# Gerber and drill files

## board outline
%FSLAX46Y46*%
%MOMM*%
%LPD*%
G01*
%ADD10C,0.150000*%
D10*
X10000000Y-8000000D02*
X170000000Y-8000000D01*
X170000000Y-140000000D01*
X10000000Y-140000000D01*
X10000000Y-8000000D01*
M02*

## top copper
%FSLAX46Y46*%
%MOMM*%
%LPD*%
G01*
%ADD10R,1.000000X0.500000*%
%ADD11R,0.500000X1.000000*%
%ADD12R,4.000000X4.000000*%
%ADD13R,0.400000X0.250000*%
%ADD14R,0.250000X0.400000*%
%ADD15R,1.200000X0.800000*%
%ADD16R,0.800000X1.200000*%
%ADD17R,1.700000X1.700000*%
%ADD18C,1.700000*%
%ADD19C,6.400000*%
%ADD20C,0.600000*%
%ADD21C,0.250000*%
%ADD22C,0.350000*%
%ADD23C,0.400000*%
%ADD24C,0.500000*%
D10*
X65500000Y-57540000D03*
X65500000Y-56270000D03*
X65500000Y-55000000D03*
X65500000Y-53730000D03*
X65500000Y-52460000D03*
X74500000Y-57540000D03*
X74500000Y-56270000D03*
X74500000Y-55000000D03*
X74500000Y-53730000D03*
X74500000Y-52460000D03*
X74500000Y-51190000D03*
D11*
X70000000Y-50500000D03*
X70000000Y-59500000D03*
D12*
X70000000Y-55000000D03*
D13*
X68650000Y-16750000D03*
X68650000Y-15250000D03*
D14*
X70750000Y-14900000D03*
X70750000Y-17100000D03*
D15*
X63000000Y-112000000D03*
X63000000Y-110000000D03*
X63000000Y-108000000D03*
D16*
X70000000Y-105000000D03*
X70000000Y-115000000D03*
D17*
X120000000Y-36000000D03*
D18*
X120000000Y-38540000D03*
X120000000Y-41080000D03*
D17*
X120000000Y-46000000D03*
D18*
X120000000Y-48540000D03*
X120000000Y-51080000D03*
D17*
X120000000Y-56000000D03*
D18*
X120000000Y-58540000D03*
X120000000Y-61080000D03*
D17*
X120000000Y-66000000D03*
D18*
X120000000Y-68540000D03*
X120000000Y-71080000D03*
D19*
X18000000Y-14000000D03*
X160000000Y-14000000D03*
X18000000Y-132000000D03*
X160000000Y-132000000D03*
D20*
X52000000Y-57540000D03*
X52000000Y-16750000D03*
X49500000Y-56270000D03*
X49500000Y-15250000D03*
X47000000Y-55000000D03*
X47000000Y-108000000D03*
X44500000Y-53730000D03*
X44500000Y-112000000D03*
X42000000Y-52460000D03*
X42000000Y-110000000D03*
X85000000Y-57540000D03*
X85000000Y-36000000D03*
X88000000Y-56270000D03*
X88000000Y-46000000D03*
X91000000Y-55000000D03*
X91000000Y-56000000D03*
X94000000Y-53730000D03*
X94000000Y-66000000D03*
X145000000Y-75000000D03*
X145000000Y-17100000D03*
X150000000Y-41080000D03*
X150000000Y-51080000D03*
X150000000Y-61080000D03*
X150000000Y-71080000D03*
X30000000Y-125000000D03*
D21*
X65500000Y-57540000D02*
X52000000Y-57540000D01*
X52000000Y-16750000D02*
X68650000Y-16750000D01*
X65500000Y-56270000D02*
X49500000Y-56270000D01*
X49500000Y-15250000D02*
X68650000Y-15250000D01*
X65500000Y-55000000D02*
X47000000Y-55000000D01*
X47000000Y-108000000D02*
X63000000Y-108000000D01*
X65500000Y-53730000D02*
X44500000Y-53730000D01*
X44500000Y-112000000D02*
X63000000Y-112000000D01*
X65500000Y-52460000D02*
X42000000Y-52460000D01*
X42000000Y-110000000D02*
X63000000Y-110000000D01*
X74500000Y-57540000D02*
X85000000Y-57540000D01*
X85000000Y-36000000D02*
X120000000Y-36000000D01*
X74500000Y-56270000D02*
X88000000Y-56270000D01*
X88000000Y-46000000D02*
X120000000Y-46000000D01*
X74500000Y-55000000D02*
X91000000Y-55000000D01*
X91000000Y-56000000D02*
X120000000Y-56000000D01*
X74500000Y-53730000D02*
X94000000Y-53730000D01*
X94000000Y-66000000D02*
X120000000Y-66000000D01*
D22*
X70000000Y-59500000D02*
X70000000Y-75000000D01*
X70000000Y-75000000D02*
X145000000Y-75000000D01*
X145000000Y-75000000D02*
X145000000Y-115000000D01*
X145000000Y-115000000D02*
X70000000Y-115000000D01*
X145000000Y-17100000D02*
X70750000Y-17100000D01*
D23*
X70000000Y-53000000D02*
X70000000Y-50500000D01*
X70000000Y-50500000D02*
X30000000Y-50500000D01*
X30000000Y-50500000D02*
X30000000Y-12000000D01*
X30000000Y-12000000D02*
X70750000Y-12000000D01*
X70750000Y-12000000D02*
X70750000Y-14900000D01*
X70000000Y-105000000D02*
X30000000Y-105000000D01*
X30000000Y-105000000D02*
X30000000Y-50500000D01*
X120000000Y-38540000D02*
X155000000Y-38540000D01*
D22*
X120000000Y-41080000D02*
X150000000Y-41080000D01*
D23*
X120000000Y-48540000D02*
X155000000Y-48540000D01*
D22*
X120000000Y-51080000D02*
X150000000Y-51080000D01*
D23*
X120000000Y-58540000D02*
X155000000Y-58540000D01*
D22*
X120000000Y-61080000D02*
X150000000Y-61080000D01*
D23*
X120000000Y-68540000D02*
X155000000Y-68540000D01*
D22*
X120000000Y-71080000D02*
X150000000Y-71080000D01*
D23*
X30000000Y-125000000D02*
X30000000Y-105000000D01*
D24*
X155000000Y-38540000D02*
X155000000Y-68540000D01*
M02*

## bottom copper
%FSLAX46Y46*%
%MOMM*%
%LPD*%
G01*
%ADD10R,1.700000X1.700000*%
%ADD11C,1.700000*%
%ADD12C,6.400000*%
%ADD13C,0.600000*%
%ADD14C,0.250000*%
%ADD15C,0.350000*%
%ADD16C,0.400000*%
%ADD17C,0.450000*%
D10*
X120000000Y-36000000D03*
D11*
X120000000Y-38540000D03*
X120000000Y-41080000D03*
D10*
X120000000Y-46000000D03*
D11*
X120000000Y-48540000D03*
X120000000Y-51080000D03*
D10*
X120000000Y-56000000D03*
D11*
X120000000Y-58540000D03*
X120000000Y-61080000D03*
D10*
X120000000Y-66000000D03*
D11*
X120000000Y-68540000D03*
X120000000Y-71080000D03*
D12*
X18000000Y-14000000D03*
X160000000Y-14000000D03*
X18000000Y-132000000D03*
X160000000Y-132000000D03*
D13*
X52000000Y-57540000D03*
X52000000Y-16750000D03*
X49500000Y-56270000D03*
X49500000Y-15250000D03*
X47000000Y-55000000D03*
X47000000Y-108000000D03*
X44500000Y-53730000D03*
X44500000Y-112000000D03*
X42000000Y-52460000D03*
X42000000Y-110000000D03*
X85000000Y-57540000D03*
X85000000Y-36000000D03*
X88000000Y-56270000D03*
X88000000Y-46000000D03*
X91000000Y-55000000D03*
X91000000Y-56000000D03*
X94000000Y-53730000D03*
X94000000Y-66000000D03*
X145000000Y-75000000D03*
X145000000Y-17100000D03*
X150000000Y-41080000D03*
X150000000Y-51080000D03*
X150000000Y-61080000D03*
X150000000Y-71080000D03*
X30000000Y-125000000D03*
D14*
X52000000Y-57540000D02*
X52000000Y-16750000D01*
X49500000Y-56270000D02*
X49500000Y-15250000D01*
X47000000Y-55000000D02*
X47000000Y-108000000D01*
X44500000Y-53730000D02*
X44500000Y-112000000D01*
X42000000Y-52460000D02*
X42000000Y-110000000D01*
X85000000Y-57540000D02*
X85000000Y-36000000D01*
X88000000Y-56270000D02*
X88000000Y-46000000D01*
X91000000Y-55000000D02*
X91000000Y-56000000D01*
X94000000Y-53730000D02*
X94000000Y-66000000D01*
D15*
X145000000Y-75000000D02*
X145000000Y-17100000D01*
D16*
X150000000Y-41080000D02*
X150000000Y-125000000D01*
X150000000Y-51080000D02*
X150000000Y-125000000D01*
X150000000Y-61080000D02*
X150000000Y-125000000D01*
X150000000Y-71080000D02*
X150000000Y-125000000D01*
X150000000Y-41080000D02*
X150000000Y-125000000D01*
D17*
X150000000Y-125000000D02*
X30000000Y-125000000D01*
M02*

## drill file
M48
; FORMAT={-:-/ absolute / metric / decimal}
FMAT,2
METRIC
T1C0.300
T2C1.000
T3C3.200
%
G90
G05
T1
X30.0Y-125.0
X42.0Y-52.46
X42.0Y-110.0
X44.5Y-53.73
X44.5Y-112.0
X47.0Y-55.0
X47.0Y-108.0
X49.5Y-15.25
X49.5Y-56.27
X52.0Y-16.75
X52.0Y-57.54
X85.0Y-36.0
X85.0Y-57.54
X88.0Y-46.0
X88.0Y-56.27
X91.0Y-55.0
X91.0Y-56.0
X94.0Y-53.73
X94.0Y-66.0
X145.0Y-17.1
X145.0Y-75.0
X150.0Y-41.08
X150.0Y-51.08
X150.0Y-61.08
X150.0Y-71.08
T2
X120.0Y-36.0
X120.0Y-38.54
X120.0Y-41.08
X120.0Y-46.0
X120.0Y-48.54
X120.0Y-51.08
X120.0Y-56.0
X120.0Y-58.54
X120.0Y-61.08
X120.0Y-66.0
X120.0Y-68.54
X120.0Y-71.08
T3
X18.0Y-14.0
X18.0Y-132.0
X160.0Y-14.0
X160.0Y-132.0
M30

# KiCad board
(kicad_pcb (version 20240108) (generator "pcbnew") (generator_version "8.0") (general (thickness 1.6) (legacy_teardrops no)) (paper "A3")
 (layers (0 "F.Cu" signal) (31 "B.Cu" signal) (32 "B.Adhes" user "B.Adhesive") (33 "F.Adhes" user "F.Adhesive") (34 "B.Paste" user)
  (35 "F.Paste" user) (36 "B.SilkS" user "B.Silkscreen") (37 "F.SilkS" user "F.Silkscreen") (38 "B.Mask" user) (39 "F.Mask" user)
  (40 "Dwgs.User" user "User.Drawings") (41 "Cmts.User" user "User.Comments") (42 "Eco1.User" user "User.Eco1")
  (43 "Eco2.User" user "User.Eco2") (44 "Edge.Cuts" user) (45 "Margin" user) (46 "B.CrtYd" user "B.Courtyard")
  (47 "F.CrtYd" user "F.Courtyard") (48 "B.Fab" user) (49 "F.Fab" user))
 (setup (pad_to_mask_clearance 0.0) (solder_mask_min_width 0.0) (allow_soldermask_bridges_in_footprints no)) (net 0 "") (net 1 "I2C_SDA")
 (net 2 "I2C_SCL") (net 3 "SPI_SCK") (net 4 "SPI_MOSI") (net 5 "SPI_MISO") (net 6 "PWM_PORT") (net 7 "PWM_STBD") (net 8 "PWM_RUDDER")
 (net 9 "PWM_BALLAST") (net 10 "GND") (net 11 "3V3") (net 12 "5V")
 (gr_rect (start 10 8) (end 170 140) (stroke (width 0.15) (type solid)) (fill none) (layer "Edge.Cuts"))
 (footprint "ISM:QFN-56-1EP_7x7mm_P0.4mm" (layer "F.Cu") (at 70 55)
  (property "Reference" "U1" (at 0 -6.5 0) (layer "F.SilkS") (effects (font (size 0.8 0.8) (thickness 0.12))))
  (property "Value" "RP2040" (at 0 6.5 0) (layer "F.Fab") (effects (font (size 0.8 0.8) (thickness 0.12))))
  (pad "1" smd rect (at -4.5 2.54) (size 1.0 0.5) (layers "F.Cu" "F.Paste" "F.Mask") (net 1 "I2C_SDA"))
  (pad "2" smd rect (at -4.5 1.27) (size 1.0 0.5) (layers "F.Cu" "F.Paste" "F.Mask") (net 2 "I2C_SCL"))
  (pad "3" smd rect (at -4.5 0) (size 1.0 0.5) (layers "F.Cu" "F.Paste" "F.Mask") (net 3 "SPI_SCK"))
  (pad "4" smd rect (at -4.5 -1.27) (size 1.0 0.5) (layers "F.Cu" "F.Paste" "F.Mask") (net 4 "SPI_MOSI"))
  (pad "5" smd rect (at -4.5 -2.54) (size 1.0 0.5) (layers "F.Cu" "F.Paste" "F.Mask") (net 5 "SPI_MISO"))
  (pad "6" smd rect (at 4.5 2.54) (size 1.0 0.5) (layers "F.Cu" "F.Paste" "F.Mask") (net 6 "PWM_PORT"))
  (pad "7" smd rect (at 4.5 1.27) (size 1.0 0.5) (layers "F.Cu" "F.Paste" "F.Mask") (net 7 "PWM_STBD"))
  (pad "8" smd rect (at 4.5 0) (size 1.0 0.5) (layers "F.Cu" "F.Paste" "F.Mask") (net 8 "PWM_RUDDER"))
  (pad "9" smd rect (at 4.5 -1.27) (size 1.0 0.5) (layers "F.Cu" "F.Paste" "F.Mask") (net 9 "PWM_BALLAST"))
  (pad "12" smd rect (at 4.5 -2.54) (size 1.0 0.5) (layers "F.Cu" "F.Paste" "F.Mask"))
  (pad "13" smd rect (at 4.5 -3.81) (size 1.0 0.5) (layers "F.Cu" "F.Paste" "F.Mask"))
  (pad "10" smd rect (at 0 -4.5) (size 0.5 1.0) (layers "F.Cu" "F.Paste" "F.Mask") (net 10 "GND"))
  (pad "11" smd rect (at 0 4.5) (size 0.5 1.0) (layers "F.Cu" "F.Paste" "F.Mask") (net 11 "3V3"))
  (pad "EP" smd rect (at 0 0) (size 4 4) (layers "F.Cu" "F.Paste" "F.Mask") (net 10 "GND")))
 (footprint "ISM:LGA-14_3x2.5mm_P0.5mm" (layer "F.Cu") (at 70 16)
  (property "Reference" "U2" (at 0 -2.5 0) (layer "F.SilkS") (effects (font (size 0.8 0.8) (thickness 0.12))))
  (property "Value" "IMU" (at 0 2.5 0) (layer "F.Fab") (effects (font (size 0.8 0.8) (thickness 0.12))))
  (pad "1" smd rect (at -1.35 0.75) (size 0.4 0.25) (layers "F.Cu" "F.Paste" "F.Mask") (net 1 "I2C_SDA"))
  (pad "2" smd rect (at -1.35 -0.75) (size 0.4 0.25) (layers "F.Cu" "F.Paste" "F.Mask") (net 2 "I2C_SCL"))
  (pad "3" smd rect (at 0.75 -1.1) (size 0.25 0.4) (layers "F.Cu" "F.Paste" "F.Mask") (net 10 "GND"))
  (pad "4" smd rect (at 0.75 1.1) (size 0.25 0.4) (layers "F.Cu" "F.Paste" "F.Mask") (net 11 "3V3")))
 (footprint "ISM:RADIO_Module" (layer "F.Cu") (at 70 110)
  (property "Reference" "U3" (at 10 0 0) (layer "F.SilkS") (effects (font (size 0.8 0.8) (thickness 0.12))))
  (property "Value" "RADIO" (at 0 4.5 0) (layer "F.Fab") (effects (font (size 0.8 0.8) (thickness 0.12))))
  (pad "1" smd rect (at -7 2) (size 1.2 0.8) (layers "F.Cu" "F.Paste" "F.Mask") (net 4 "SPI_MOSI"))
  (pad "2" smd rect (at -7 0) (size 1.2 0.8) (layers "F.Cu" "F.Paste" "F.Mask") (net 5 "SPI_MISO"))
  (pad "3" smd rect (at -7 -2) (size 1.2 0.8) (layers "F.Cu" "F.Paste" "F.Mask") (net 3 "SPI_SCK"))
  (pad "4" smd rect (at 0 -5) (size 0.8 1.2) (layers "F.Cu" "F.Paste" "F.Mask") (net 10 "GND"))
  (pad "5" smd rect (at 0 5) (size 0.8 1.2) (layers "F.Cu" "F.Paste" "F.Mask") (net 11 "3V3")))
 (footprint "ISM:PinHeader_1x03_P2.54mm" (layer "F.Cu") (at 120 36)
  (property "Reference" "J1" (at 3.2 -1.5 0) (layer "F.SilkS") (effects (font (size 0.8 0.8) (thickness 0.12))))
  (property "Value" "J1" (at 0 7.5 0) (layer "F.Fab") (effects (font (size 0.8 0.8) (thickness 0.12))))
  (pad "1" thru_hole rect (at 0 0) (size 1.7 1.7) (drill 1.0) (layers "*.Cu" "*.Mask") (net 6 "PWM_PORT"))
  (pad "2" thru_hole circle (at 0 2.54) (size 1.7 1.7) (drill 1.0) (layers "*.Cu" "*.Mask") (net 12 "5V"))
  (pad "3" thru_hole circle (at 0 5.08) (size 1.7 1.7) (drill 1.0) (layers "*.Cu" "*.Mask") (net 10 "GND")))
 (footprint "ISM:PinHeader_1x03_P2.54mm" (layer "F.Cu") (at 120 46)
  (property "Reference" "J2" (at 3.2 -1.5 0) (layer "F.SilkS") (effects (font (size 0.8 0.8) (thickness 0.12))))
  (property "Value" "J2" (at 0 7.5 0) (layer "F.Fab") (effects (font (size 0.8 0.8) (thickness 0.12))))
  (pad "1" thru_hole rect (at 0 0) (size 1.7 1.7) (drill 1.0) (layers "*.Cu" "*.Mask") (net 7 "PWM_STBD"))
  (pad "2" thru_hole circle (at 0 2.54) (size 1.7 1.7) (drill 1.0) (layers "*.Cu" "*.Mask") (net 12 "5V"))
  (pad "3" thru_hole circle (at 0 5.08) (size 1.7 1.7) (drill 1.0) (layers "*.Cu" "*.Mask") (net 10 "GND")))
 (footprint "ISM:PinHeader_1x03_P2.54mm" (layer "F.Cu") (at 120 56)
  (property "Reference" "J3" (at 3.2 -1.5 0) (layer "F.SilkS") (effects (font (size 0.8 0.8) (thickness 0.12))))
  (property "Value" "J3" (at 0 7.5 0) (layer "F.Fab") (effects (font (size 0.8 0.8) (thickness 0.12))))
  (pad "1" thru_hole rect (at 0 0) (size 1.7 1.7) (drill 1.0) (layers "*.Cu" "*.Mask") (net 8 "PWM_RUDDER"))
  (pad "2" thru_hole circle (at 0 2.54) (size 1.7 1.7) (drill 1.0) (layers "*.Cu" "*.Mask") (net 12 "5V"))
  (pad "3" thru_hole circle (at 0 5.08) (size 1.7 1.7) (drill 1.0) (layers "*.Cu" "*.Mask") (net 10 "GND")))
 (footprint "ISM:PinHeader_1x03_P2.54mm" (layer "F.Cu") (at 120 66)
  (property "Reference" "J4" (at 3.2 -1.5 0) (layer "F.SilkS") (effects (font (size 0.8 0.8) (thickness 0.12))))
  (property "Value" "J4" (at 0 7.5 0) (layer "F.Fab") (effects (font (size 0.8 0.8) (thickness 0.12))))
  (pad "1" thru_hole rect (at 0 0) (size 1.7 1.7) (drill 1.0) (layers "*.Cu" "*.Mask") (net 9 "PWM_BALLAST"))
  (pad "2" thru_hole circle (at 0 2.54) (size 1.7 1.7) (drill 1.0) (layers "*.Cu" "*.Mask") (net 12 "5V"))
  (pad "3" thru_hole circle (at 0 5.08) (size 1.7 1.7) (drill 1.0) (layers "*.Cu" "*.Mask") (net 10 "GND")))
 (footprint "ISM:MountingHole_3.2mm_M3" (layer "F.Cu") (at 18 14)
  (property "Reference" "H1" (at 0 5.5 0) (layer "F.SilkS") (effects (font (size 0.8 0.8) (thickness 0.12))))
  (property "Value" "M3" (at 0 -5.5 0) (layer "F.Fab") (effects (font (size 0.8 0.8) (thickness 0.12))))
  (pad "" thru_hole circle (at 0 0) (size 6.4 6.4) (drill 3.2) (layers "*.Cu" "*.Mask")))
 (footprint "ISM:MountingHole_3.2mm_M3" (layer "F.Cu") (at 160 14)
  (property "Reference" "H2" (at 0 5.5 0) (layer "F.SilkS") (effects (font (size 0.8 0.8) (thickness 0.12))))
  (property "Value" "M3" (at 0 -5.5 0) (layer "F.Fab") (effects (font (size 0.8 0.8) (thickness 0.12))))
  (pad "" thru_hole circle (at 0 0) (size 6.4 6.4) (drill 3.2) (layers "*.Cu" "*.Mask")))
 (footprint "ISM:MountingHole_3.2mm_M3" (layer "F.Cu") (at 18 132)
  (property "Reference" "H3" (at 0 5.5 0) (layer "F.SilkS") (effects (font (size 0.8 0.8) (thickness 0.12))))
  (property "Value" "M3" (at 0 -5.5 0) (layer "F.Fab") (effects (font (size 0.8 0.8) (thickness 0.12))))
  (pad "" thru_hole circle (at 0 0) (size 6.4 6.4) (drill 3.2) (layers "*.Cu" "*.Mask")))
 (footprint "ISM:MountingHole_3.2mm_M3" (layer "F.Cu") (at 160 132)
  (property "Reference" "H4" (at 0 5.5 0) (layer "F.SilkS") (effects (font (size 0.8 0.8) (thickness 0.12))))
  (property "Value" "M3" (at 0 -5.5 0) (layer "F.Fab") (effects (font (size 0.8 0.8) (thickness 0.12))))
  (pad "" thru_hole circle (at 0 0) (size 6.4 6.4) (drill 3.2) (layers "*.Cu" "*.Mask")))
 (segment (start 65.5 57.54) (end 52.0 57.54) (width 0.25) (layer "F.Cu") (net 1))
 (segment (start 52.0 57.54) (end 52.0 16.75) (width 0.25) (layer "B.Cu") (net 1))
 (segment (start 52.0 16.75) (end 68.65 16.75) (width 0.25) (layer "F.Cu") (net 1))
 (segment (start 65.5 56.27) (end 49.5 56.27) (width 0.25) (layer "F.Cu") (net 2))
 (segment (start 49.5 56.27) (end 49.5 15.25) (width 0.25) (layer "B.Cu") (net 2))
 (segment (start 49.5 15.25) (end 68.65 15.25) (width 0.25) (layer "F.Cu") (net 2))
 (segment (start 65.5 55) (end 47.0 55) (width 0.25) (layer "F.Cu") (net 3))
 (segment (start 47.0 55) (end 47.0 108) (width 0.25) (layer "B.Cu") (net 3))
 (segment (start 47.0 108) (end 63 108) (width 0.25) (layer "F.Cu") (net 3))
 (segment (start 65.5 53.73) (end 44.5 53.73) (width 0.25) (layer "F.Cu") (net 4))
 (segment (start 44.5 53.73) (end 44.5 112) (width 0.25) (layer "B.Cu") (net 4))
 (segment (start 44.5 112) (end 63 112) (width 0.25) (layer "F.Cu") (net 4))
 (segment (start 65.5 52.46) (end 42.0 52.46) (width 0.25) (layer "F.Cu") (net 5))
 (segment (start 42.0 52.46) (end 42.0 110) (width 0.25) (layer "B.Cu") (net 5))
 (segment (start 42.0 110) (end 63 110) (width 0.25) (layer "F.Cu") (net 5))
 (segment (start 74.5 57.54) (end 85 57.54) (width 0.25) (layer "F.Cu") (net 6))
 (segment (start 85 57.54) (end 85 36) (width 0.25) (layer "B.Cu") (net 6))
 (segment (start 85 36) (end 120 36) (width 0.25) (layer "F.Cu") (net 6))
 (segment (start 74.5 56.27) (end 88 56.27) (width 0.25) (layer "F.Cu") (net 7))
 (segment (start 88 56.27) (end 88 46) (width 0.25) (layer "B.Cu") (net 7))
 (segment (start 88 46) (end 120 46) (width 0.25) (layer "F.Cu") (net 7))
 (segment (start 74.5 55) (end 91 55) (width 0.25) (layer "F.Cu") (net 8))
 (segment (start 91 55) (end 91 56) (width 0.25) (layer "B.Cu") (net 8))
 (segment (start 91 56) (end 120 56) (width 0.25) (layer "F.Cu") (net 8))
 (segment (start 74.5 53.73) (end 94 53.73) (width 0.25) (layer "F.Cu") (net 9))
 (segment (start 94 53.73) (end 94 66) (width 0.25) (layer "B.Cu") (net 9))
 (segment (start 94 66) (end 120 66) (width 0.25) (layer "F.Cu") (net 9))
 (segment (start 70 59.5) (end 70 75) (width 0.35) (layer "F.Cu") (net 11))
 (segment (start 70 75) (end 145 75) (width 0.35) (layer "F.Cu") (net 11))
 (segment (start 145 75) (end 145 115) (width 0.35) (layer "F.Cu") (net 11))
 (segment (start 145 115) (end 70 115) (width 0.35) (layer "F.Cu") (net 11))
 (segment (start 145 75) (end 145 17.1) (width 0.35) (layer "B.Cu") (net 11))
 (segment (start 145 17.1) (end 70.75 17.1) (width 0.35) (layer "F.Cu") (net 11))
 (segment (start 70 53) (end 70 50.5) (width 0.4) (layer "F.Cu") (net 10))
 (segment (start 70 50.5) (end 30 50.5) (width 0.4) (layer "F.Cu") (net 10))
 (segment (start 30 50.5) (end 30 12) (width 0.4) (layer "F.Cu") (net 10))
 (segment (start 30 12) (end 70.75 12) (width 0.4) (layer "F.Cu") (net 10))
 (segment (start 70.75 12) (end 70.75 14.9) (width 0.4) (layer "F.Cu") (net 10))
 (segment (start 70 105) (end 30 105) (width 0.4) (layer "F.Cu") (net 10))
 (segment (start 30 105) (end 30 50.5) (width 0.4) (layer "F.Cu") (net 10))
 (segment (start 120 38.54) (end 155 38.54) (width 0.4) (layer "F.Cu") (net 12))
 (segment (start 120 41.08) (end 150 41.08) (width 0.35) (layer "F.Cu") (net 10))
 (segment (start 150 41.08) (end 150 125) (width 0.4) (layer "B.Cu") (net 10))
 (segment (start 120 48.54) (end 155 48.54) (width 0.4) (layer "F.Cu") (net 12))
 (segment (start 120 51.08) (end 150 51.08) (width 0.35) (layer "F.Cu") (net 10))
 (segment (start 150 51.08) (end 150 125) (width 0.4) (layer "B.Cu") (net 10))
 (segment (start 120 58.54) (end 155 58.54) (width 0.4) (layer "F.Cu") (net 12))
 (segment (start 120 61.08) (end 150 61.08) (width 0.35) (layer "F.Cu") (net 10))
 (segment (start 150 61.08) (end 150 125) (width 0.4) (layer "B.Cu") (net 10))
 (segment (start 120 68.54) (end 155 68.54) (width 0.4) (layer "F.Cu") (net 12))
 (segment (start 120 71.08) (end 150 71.08) (width 0.35) (layer "F.Cu") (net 10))
 (segment (start 150 71.08) (end 150 125) (width 0.4) (layer "B.Cu") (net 10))
 (segment (start 150 41.08) (end 150 125) (width 0.4) (layer "B.Cu") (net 10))
 (segment (start 150 125) (end 30 125) (width 0.45) (layer "B.Cu") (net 10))
 (segment (start 30 125) (end 30 105) (width 0.4) (layer "F.Cu") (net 10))
 (segment (start 155 38.54) (end 155 68.54) (width 0.5) (layer "F.Cu") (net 12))
 (via (at 52.0 57.54) (size 0.6) (drill 0.3) (layers "F.Cu" "B.Cu") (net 1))
 (via (at 52.0 16.75) (size 0.6) (drill 0.3) (layers "F.Cu" "B.Cu") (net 1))
 (via (at 49.5 56.27) (size 0.6) (drill 0.3) (layers "F.Cu" "B.Cu") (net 2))
 (via (at 49.5 15.25) (size 0.6) (drill 0.3) (layers "F.Cu" "B.Cu") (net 2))
 (via (at 47.0 55) (size 0.6) (drill 0.3) (layers "F.Cu" "B.Cu") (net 3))
 (via (at 47.0 108) (size 0.6) (drill 0.3) (layers "F.Cu" "B.Cu") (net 3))
 (via (at 44.5 53.73) (size 0.6) (drill 0.3) (layers "F.Cu" "B.Cu") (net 4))
 (via (at 44.5 112) (size 0.6) (drill 0.3) (layers "F.Cu" "B.Cu") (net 4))
 (via (at 42.0 52.46) (size 0.6) (drill 0.3) (layers "F.Cu" "B.Cu") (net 5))
 (via (at 42.0 110) (size 0.6) (drill 0.3) (layers "F.Cu" "B.Cu") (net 5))
 (via (at 85 57.54) (size 0.6) (drill 0.3) (layers "F.Cu" "B.Cu") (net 6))
 (via (at 85 36) (size 0.6) (drill 0.3) (layers "F.Cu" "B.Cu") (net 6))
 (via (at 88 56.27) (size 0.6) (drill 0.3) (layers "F.Cu" "B.Cu") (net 7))
 (via (at 88 46) (size 0.6) (drill 0.3) (layers "F.Cu" "B.Cu") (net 7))
 (via (at 91 55) (size 0.6) (drill 0.3) (layers "F.Cu" "B.Cu") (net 8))
 (via (at 91 56) (size 0.6) (drill 0.3) (layers "F.Cu" "B.Cu") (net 8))
 (via (at 94 53.73) (size 0.6) (drill 0.3) (layers "F.Cu" "B.Cu") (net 9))
 (via (at 94 66) (size 0.6) (drill 0.3) (layers "F.Cu" "B.Cu") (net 9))
 (via (at 145 75) (size 0.6) (drill 0.3) (layers "F.Cu" "B.Cu") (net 11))
 (via (at 145 17.1) (size 0.6) (drill 0.3) (layers "F.Cu" "B.Cu") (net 11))
 (via (at 150 41.08) (size 0.6) (drill 0.3) (layers "F.Cu" "B.Cu") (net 10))
 (via (at 150 51.08) (size 0.6) (drill 0.3) (layers "F.Cu" "B.Cu") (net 10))
 (via (at 150 61.08) (size 0.6) (drill 0.3) (layers "F.Cu" "B.Cu") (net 10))
 (via (at 150 71.08) (size 0.6) (drill 0.3) (layers "F.Cu" "B.Cu") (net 10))
 (via (at 30 125) (size 0.6) (drill 0.3) (layers "F.Cu" "B.Cu") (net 10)))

